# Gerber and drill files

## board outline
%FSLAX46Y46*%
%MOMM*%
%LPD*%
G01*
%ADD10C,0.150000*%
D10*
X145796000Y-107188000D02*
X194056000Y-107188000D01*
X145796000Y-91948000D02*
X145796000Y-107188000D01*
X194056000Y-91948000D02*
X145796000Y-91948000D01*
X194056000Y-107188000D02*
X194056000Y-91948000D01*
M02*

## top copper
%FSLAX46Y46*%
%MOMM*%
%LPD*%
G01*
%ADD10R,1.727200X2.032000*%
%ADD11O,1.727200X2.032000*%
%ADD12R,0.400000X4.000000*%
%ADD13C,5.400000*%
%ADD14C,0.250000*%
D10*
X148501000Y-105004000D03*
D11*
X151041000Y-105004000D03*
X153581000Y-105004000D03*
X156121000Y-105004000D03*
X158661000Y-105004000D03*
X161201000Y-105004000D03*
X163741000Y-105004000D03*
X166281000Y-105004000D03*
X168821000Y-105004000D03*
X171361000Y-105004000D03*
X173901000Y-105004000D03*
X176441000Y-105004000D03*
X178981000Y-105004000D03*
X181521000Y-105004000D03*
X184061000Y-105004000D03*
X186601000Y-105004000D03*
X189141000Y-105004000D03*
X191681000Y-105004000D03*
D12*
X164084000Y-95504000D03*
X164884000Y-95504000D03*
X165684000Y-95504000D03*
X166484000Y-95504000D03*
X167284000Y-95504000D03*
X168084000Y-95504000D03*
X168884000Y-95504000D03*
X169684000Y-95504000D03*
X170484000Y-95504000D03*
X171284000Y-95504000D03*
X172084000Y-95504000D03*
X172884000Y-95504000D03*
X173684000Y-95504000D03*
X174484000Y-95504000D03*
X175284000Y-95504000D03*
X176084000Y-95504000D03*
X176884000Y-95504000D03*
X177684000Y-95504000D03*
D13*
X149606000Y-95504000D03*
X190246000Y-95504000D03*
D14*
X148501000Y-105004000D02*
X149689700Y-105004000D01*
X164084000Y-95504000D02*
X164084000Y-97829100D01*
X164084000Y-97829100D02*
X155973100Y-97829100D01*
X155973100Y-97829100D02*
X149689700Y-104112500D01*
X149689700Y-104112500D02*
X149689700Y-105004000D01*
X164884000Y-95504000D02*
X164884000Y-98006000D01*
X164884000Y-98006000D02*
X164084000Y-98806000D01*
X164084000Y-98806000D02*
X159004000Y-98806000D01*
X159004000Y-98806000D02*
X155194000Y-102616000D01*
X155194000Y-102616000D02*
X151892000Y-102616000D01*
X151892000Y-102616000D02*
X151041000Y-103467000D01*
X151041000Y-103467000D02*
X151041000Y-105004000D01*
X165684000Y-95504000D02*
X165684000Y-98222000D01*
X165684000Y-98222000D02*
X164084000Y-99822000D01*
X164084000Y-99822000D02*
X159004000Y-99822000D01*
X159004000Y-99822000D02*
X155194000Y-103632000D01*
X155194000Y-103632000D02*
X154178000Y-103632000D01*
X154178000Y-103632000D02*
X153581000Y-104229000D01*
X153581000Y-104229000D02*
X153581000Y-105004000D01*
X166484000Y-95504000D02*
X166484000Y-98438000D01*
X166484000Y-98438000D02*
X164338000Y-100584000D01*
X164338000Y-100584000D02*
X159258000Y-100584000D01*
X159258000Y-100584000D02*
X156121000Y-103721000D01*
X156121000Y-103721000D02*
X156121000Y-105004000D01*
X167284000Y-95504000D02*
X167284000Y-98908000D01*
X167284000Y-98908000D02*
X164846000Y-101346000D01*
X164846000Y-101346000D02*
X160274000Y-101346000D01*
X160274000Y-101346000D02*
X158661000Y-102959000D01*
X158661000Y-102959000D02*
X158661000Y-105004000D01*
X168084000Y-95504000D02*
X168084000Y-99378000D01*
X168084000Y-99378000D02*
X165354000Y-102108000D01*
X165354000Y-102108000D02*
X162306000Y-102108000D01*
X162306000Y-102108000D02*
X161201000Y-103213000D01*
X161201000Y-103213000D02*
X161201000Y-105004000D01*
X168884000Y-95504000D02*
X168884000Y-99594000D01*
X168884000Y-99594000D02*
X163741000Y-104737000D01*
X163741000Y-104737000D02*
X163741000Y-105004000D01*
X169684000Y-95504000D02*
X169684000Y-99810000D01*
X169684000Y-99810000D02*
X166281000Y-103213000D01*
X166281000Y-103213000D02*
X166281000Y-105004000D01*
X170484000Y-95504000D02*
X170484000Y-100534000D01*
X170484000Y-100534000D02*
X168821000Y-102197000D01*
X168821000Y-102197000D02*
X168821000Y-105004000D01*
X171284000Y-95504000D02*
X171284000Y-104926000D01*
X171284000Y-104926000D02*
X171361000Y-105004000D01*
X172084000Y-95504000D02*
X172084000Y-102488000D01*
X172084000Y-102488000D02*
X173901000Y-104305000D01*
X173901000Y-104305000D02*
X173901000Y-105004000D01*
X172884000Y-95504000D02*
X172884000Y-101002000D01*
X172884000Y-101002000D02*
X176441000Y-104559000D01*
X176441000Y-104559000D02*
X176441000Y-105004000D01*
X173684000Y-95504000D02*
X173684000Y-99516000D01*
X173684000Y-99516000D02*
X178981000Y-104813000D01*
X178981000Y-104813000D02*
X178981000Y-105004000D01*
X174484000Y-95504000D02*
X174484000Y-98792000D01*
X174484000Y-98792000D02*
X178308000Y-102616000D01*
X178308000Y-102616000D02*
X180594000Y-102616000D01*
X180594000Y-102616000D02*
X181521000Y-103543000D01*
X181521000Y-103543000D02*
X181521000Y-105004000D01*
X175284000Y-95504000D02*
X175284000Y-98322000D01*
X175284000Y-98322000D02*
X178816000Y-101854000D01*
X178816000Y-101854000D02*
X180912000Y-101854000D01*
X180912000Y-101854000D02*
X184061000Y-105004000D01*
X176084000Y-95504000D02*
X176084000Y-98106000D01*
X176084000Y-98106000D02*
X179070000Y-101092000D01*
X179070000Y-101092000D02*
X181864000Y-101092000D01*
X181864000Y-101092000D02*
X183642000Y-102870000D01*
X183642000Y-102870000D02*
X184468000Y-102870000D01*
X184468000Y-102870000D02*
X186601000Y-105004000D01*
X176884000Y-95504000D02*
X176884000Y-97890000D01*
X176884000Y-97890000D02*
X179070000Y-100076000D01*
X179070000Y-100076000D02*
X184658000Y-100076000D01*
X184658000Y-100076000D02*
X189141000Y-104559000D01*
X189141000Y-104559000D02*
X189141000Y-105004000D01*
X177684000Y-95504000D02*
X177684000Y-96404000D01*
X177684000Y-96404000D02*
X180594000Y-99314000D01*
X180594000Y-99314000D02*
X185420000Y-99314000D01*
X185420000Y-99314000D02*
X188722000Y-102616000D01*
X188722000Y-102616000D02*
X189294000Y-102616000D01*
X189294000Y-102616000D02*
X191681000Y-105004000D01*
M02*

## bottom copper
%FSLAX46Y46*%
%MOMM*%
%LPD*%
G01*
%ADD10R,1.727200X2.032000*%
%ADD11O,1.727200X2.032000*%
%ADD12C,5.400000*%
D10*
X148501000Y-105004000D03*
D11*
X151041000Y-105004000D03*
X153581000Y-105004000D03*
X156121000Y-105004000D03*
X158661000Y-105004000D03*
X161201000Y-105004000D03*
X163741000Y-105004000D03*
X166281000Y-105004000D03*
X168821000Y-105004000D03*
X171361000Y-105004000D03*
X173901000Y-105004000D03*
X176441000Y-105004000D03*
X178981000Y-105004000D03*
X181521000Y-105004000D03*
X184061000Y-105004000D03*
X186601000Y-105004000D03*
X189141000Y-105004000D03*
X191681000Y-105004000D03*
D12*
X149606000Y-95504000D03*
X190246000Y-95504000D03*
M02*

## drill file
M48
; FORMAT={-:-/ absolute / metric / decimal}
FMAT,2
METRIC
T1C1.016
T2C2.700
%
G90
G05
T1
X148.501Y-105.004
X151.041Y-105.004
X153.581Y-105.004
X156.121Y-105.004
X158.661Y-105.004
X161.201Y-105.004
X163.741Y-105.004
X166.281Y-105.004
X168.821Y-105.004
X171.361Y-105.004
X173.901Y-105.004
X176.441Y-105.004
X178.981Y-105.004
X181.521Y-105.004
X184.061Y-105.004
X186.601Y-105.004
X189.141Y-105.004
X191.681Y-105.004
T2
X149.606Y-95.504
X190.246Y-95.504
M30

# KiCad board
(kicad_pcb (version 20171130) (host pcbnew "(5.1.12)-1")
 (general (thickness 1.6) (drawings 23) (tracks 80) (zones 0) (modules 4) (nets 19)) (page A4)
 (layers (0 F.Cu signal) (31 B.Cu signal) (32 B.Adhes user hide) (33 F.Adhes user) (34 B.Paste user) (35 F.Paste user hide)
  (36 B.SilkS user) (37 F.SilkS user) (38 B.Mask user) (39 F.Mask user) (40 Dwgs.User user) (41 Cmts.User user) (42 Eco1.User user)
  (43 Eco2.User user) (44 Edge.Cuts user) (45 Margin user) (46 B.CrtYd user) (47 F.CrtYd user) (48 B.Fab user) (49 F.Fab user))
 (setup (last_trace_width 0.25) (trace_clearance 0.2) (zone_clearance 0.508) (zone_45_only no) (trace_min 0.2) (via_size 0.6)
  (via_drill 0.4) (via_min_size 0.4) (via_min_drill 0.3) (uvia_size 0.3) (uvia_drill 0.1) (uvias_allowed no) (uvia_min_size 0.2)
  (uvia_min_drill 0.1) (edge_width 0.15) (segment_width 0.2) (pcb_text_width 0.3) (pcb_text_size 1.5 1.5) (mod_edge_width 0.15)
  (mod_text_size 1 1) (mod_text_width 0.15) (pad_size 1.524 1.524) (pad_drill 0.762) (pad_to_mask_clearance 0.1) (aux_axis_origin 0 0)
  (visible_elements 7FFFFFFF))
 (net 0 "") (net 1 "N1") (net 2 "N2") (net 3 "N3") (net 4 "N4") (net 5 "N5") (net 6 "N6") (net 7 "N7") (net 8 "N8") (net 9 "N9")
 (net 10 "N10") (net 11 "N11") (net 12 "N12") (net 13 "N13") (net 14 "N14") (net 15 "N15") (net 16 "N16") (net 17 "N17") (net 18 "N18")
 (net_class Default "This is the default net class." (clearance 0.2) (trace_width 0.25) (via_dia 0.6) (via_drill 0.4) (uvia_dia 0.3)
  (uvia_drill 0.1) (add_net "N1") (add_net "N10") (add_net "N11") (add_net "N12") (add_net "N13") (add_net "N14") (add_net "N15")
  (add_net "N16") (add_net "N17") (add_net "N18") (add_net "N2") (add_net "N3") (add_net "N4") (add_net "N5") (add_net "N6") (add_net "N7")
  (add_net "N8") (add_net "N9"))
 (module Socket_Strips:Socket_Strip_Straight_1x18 (layer F.Cu) (at 148.501 105.004)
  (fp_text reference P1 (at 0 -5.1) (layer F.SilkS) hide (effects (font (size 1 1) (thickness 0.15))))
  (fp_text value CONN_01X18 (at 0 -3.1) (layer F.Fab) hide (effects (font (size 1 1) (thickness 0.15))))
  (pad 1 thru_hole rect (at 0 0) (size 1.7272 2.032) (drill 1.016) (layers *.Cu *.Mask) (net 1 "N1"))
  (pad 2 thru_hole oval (at 2.54 0) (size 1.7272 2.032) (drill 1.016) (layers *.Cu *.Mask) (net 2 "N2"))
  (pad 3 thru_hole oval (at 5.08 0) (size 1.7272 2.032) (drill 1.016) (layers *.Cu *.Mask) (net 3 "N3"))
  (pad 4 thru_hole oval (at 7.62 0) (size 1.7272 2.032) (drill 1.016) (layers *.Cu *.Mask) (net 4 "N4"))
  (pad 5 thru_hole oval (at 10.16 0) (size 1.7272 2.032) (drill 1.016) (layers *.Cu *.Mask) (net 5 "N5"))
  (pad 6 thru_hole oval (at 12.7 0) (size 1.7272 2.032) (drill 1.016) (layers *.Cu *.Mask) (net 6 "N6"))
  (pad 7 thru_hole oval (at 15.24 0) (size 1.7272 2.032) (drill 1.016) (layers *.Cu *.Mask) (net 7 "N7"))
  (pad 8 thru_hole oval (at 17.78 0) (size 1.7272 2.032) (drill 1.016) (layers *.Cu *.Mask) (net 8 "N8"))
  (pad 9 thru_hole oval (at 20.32 0) (size 1.7272 2.032) (drill 1.016) (layers *.Cu *.Mask) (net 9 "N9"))
  (pad 10 thru_hole oval (at 22.86 0) (size 1.7272 2.032) (drill 1.016) (layers *.Cu *.Mask) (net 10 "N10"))
  (pad 11 thru_hole oval (at 25.4 0) (size 1.7272 2.032) (drill 1.016) (layers *.Cu *.Mask) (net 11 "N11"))
  (pad 12 thru_hole oval (at 27.94 0) (size 1.7272 2.032) (drill 1.016) (layers *.Cu *.Mask) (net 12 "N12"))
  (pad 13 thru_hole oval (at 30.48 0) (size 1.7272 2.032) (drill 1.016) (layers *.Cu *.Mask) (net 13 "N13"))
  (pad 14 thru_hole oval (at 33.02 0) (size 1.7272 2.032) (drill 1.016) (layers *.Cu *.Mask) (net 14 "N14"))
  (pad 15 thru_hole oval (at 35.56 0) (size 1.7272 2.032) (drill 1.016) (layers *.Cu *.Mask) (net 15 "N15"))
  (pad 16 thru_hole oval (at 38.1 0) (size 1.7272 2.032) (drill 1.016) (layers *.Cu *.Mask) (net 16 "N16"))
  (pad 17 thru_hole oval (at 40.64 0) (size 1.7272 2.032) (drill 1.016) (layers *.Cu *.Mask) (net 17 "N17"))
  (pad 18 thru_hole oval (at 43.18 0) (size 1.7272 2.032) (drill 1.016) (layers *.Cu *.Mask) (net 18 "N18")))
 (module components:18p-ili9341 (layer F.Cu) (at 164.084 95.504)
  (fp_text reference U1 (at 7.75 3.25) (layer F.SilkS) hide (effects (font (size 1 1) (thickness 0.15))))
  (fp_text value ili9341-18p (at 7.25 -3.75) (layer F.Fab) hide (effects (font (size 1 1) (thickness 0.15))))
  (pad 1 smd rect (at 0 0) (size 0.4 4) (layers F.Cu F.Paste F.Mask) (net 1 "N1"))
  (pad 2 smd rect (at 0.8 0) (size 0.4 4) (layers F.Cu F.Paste F.Mask) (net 2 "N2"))
  (pad 3 smd rect (at 1.6 0) (size 0.4 4) (layers F.Cu F.Paste F.Mask) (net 3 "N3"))
  (pad 4 smd rect (at 2.4 0) (size 0.4 4) (layers F.Cu F.Paste F.Mask) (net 4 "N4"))
  (pad 5 smd rect (at 3.2 0) (size 0.4 4) (layers F.Cu F.Paste F.Mask) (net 5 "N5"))
  (pad 6 smd rect (at 4 0) (size 0.4 4) (layers F.Cu F.Paste F.Mask) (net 6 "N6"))
  (pad 7 smd rect (at 4.8 0) (size 0.4 4) (layers F.Cu F.Paste F.Mask) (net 7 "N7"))
  (pad 8 smd rect (at 5.6 0) (size 0.4 4) (layers F.Cu F.Paste F.Mask) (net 8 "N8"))
  (pad 9 smd rect (at 6.4 0) (size 0.4 4) (layers F.Cu F.Paste F.Mask) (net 9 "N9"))
  (pad 10 smd rect (at 7.2 0) (size 0.4 4) (layers F.Cu F.Paste F.Mask) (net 10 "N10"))
  (pad 11 smd rect (at 8 0) (size 0.4 4) (layers F.Cu F.Paste F.Mask) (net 11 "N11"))
  (pad 12 smd rect (at 8.8 0) (size 0.4 4) (layers F.Cu F.Paste F.Mask) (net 12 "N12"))
  (pad 13 smd rect (at 9.6 0) (size 0.4 4) (layers F.Cu F.Paste F.Mask) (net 13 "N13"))
  (pad 14 smd rect (at 10.4 0) (size 0.4 4) (layers F.Cu F.Paste F.Mask) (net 14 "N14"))
  (pad 15 smd rect (at 11.2 0) (size 0.4 4) (layers F.Cu F.Paste F.Mask) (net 15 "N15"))
  (pad 16 smd rect (at 12 0) (size 0.4 4) (layers F.Cu F.Paste F.Mask) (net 16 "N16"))
  (pad 17 smd rect (at 12.8 0) (size 0.4 4) (layers F.Cu F.Paste F.Mask) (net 17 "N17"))
  (pad 18 smd rect (at 13.6 0) (size 0.4 4) (layers F.Cu F.Paste F.Mask) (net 18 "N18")))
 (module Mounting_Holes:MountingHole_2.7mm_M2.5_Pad (layer F.Cu) (at 149.606 95.504)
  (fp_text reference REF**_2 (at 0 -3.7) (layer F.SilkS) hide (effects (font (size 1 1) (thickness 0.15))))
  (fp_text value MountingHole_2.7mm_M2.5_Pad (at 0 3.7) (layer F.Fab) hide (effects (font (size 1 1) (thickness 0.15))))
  (pad 1 thru_hole circle (at 0 0) (size 5.4 5.4) (drill 2.7) (layers *.Cu *.Mask)))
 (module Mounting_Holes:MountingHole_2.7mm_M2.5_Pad (layer F.Cu) (at 190.246 95.504)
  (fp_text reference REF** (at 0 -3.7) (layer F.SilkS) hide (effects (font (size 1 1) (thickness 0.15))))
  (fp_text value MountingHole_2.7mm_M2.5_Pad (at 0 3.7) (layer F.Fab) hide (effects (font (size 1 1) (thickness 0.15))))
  (pad 1 thru_hole circle (at 0 0) (size 5.4 5.4) (drill 2.7) (layers *.Cu *.Mask)))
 (gr_line (start 145.796 107.188) (end 194.056 107.188) (angle 90) (layer Edge.Cuts) (width 0.15))
 (gr_line (start 145.796 91.948) (end 145.796 107.188) (angle 90) (layer Edge.Cuts) (width 0.15))
 (gr_line (start 194.056 91.948) (end 145.796 91.948) (angle 90) (layer Edge.Cuts) (width 0.15))
 (gr_line (start 194.056 107.188) (end 194.056 91.948) (angle 90) (layer Edge.Cuts) (width 0.15))
 (segment (start 148.501 105.004) (end 149.6897 105.004) (width 0.25) (layer F.Cu) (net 1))
 (segment (start 164.084 95.504) (end 164.084 97.8291) (width 0.25) (layer F.Cu) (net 1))
 (segment (start 164.084 97.8291) (end 155.9731 97.8291) (width 0.25) (layer F.Cu) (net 1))
 (segment (start 155.9731 97.8291) (end 149.6897 104.1125) (width 0.25) (layer F.Cu) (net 1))
 (segment (start 149.6897 104.1125) (end 149.6897 105.004) (width 0.25) (layer F.Cu) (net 1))
 (segment (start 164.884 95.504) (end 164.884 98.006) (width 0.25) (layer F.Cu) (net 2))
 (segment (start 164.884 98.006) (end 164.084 98.806) (width 0.25) (layer F.Cu) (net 2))
 (segment (start 164.084 98.806) (end 159.004 98.806) (width 0.25) (layer F.Cu) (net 2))
 (segment (start 159.004 98.806) (end 155.194 102.616) (width 0.25) (layer F.Cu) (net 2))
 (segment (start 155.194 102.616) (end 151.892 102.616) (width 0.25) (layer F.Cu) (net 2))
 (segment (start 151.892 102.616) (end 151.041 103.467) (width 0.25) (layer F.Cu) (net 2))
 (segment (start 151.041 103.467) (end 151.041 105.004) (width 0.25) (layer F.Cu) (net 2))
 (segment (start 165.684 95.504) (end 165.684 98.222) (width 0.25) (layer F.Cu) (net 3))
 (segment (start 165.684 98.222) (end 164.084 99.822) (width 0.25) (layer F.Cu) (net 3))
 (segment (start 164.084 99.822) (end 159.004 99.822) (width 0.25) (layer F.Cu) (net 3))
 (segment (start 159.004 99.822) (end 155.194 103.632) (width 0.25) (layer F.Cu) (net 3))
 (segment (start 155.194 103.632) (end 154.178 103.632) (width 0.25) (layer F.Cu) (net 3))
 (segment (start 154.178 103.632) (end 153.581 104.229) (width 0.25) (layer F.Cu) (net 3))
 (segment (start 153.581 104.229) (end 153.581 105.004) (width 0.25) (layer F.Cu) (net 3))
 (segment (start 166.484 95.504) (end 166.484 98.438) (width 0.25) (layer F.Cu) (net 4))
 (segment (start 166.484 98.438) (end 164.338 100.584) (width 0.25) (layer F.Cu) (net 4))
 (segment (start 164.338 100.584) (end 159.258 100.584) (width 0.25) (layer F.Cu) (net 4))
 (segment (start 159.258 100.584) (end 156.121 103.721) (width 0.25) (layer F.Cu) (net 4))
 (segment (start 156.121 103.721) (end 156.121 105.004) (width 0.25) (layer F.Cu) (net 4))
 (segment (start 167.284 95.504) (end 167.284 98.908) (width 0.25) (layer F.Cu) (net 5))
 (segment (start 167.284 98.908) (end 164.846 101.346) (width 0.25) (layer F.Cu) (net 5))
 (segment (start 164.846 101.346) (end 160.274 101.346) (width 0.25) (layer F.Cu) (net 5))
 (segment (start 160.274 101.346) (end 158.661 102.959) (width 0.25) (layer F.Cu) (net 5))
 (segment (start 158.661 102.959) (end 158.661 105.004) (width 0.25) (layer F.Cu) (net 5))
 (segment (start 168.084 95.504) (end 168.084 99.378) (width 0.25) (layer F.Cu) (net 6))
 (segment (start 168.084 99.378) (end 165.354 102.108) (width 0.25) (layer F.Cu) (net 6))
 (segment (start 165.354 102.108) (end 162.306 102.108) (width 0.25) (layer F.Cu) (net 6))
 (segment (start 162.306 102.108) (end 161.201 103.213) (width 0.25) (layer F.Cu) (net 6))
 (segment (start 161.201 103.213) (end 161.201 105.004) (width 0.25) (layer F.Cu) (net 6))
 (segment (start 168.884 95.504) (end 168.884 99.594) (width 0.25) (layer F.Cu) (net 7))
 (segment (start 168.884 99.594) (end 163.741 104.737) (width 0.25) (layer F.Cu) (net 7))
 (segment (start 163.741 104.737) (end 163.741 105.004) (width 0.25) (layer F.Cu) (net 7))
 (segment (start 169.684 95.504) (end 169.684 99.81) (width 0.25) (layer F.Cu) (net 8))
 (segment (start 169.684 99.81) (end 166.281 103.213) (width 0.25) (layer F.Cu) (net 8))
 (segment (start 166.281 103.213) (end 166.281 105.004) (width 0.25) (layer F.Cu) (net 8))
 (segment (start 170.484 95.504) (end 170.484 100.534) (width 0.25) (layer F.Cu) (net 9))
 (segment (start 170.484 100.534) (end 168.821 102.197) (width 0.25) (layer F.Cu) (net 9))
 (segment (start 168.821 102.197) (end 168.821 105.004) (width 0.25) (layer F.Cu) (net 9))
 (segment (start 171.284 95.504) (end 171.284 104.926) (width 0.25) (layer F.Cu) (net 10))
 (segment (start 171.284 104.926) (end 171.361 105.004) (width 0.25) (layer F.Cu) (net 10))
 (segment (start 172.084 95.504) (end 172.084 102.488) (width 0.25) (layer F.Cu) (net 11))
 (segment (start 172.084 102.488) (end 173.901 104.305) (width 0.25) (layer F.Cu) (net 11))
 (segment (start 173.901 104.305) (end 173.901 105.004) (width 0.25) (layer F.Cu) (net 11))
 (segment (start 172.884 95.504) (end 172.884 101.002) (width 0.25) (layer F.Cu) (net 12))
 (segment (start 172.884 101.002) (end 176.441 104.559) (width 0.25) (layer F.Cu) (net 12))
 (segment (start 176.441 104.559) (end 176.441 105.004) (width 0.25) (layer F.Cu) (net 12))
 (segment (start 173.684 95.504) (end 173.684 99.516) (width 0.25) (layer F.Cu) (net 13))
 (segment (start 173.684 99.516) (end 178.981 104.813) (width 0.25) (layer F.Cu) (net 13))
 (segment (start 178.981 104.813) (end 178.981 105.004) (width 0.25) (layer F.Cu) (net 13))
 (segment (start 174.484 95.504) (end 174.484 98.792) (width 0.25) (layer F.Cu) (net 14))
 (segment (start 174.484 98.792) (end 178.308 102.616) (width 0.25) (layer F.Cu) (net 14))
 (segment (start 178.308 102.616) (end 180.594 102.616) (width 0.25) (layer F.Cu) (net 14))
 (segment (start 180.594 102.616) (end 181.521 103.543) (width 0.25) (layer F.Cu) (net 14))
 (segment (start 181.521 103.543) (end 181.521 105.004) (width 0.25) (layer F.Cu) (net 14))
 (segment (start 175.284 95.504) (end 175.284 98.322) (width 0.25) (layer F.Cu) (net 15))
 (segment (start 175.284 98.322) (end 178.816 101.854) (width 0.25) (layer F.Cu) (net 15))
 (segment (start 178.816 101.854) (end 180.912 101.854) (width 0.25) (layer F.Cu) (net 15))
 (segment (start 180.912 101.854) (end 184.061 105.004) (width 0.25) (layer F.Cu) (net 15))
 (segment (start 176.084 95.504) (end 176.084 98.106) (width 0.25) (layer F.Cu) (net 16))
 (segment (start 176.084 98.106) (end 179.07 101.092) (width 0.25) (layer F.Cu) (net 16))
 (segment (start 179.07 101.092) (end 181.864 101.092) (width 0.25) (layer F.Cu) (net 16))
 (segment (start 181.864 101.092) (end 183.642 102.87) (width 0.25) (layer F.Cu) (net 16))
 (segment (start 183.642 102.87) (end 184.468 102.87) (width 0.25) (layer F.Cu) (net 16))
 (segment (start 184.468 102.87) (end 186.601 105.004) (width 0.25) (layer F.Cu) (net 16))
 (segment (start 176.884 95.504) (end 176.884 97.89) (width 0.25) (layer F.Cu) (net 17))
 (segment (start 176.884 97.89) (end 179.07 100.076) (width 0.25) (layer F.Cu) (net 17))
 (segment (start 179.07 100.076) (end 184.658 100.076) (width 0.25) (layer F.Cu) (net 17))
 (segment (start 184.658 100.076) (end 189.141 104.559) (width 0.25) (layer F.Cu) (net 17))
 (segment (start 189.141 104.559) (end 189.141 105.004) (width 0.25) (layer F.Cu) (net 17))
 (segment (start 177.684 95.504) (end 177.684 96.404) (width 0.25) (layer F.Cu) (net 18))
 (segment (start 177.684 96.404) (end 180.594 99.314) (width 0.25) (layer F.Cu) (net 18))
 (segment (start 180.594 99.314) (end 185.42 99.314) (width 0.25) (layer F.Cu) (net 18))
 (segment (start 185.42 99.314) (end 188.722 102.616) (width 0.25) (layer F.Cu) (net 18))
 (segment (start 188.722 102.616) (end 189.294 102.616) (width 0.25) (layer F.Cu) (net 18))
 (segment (start 189.294 102.616) (end 191.681 105.004) (width 0.25) (layer F.Cu) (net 18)))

